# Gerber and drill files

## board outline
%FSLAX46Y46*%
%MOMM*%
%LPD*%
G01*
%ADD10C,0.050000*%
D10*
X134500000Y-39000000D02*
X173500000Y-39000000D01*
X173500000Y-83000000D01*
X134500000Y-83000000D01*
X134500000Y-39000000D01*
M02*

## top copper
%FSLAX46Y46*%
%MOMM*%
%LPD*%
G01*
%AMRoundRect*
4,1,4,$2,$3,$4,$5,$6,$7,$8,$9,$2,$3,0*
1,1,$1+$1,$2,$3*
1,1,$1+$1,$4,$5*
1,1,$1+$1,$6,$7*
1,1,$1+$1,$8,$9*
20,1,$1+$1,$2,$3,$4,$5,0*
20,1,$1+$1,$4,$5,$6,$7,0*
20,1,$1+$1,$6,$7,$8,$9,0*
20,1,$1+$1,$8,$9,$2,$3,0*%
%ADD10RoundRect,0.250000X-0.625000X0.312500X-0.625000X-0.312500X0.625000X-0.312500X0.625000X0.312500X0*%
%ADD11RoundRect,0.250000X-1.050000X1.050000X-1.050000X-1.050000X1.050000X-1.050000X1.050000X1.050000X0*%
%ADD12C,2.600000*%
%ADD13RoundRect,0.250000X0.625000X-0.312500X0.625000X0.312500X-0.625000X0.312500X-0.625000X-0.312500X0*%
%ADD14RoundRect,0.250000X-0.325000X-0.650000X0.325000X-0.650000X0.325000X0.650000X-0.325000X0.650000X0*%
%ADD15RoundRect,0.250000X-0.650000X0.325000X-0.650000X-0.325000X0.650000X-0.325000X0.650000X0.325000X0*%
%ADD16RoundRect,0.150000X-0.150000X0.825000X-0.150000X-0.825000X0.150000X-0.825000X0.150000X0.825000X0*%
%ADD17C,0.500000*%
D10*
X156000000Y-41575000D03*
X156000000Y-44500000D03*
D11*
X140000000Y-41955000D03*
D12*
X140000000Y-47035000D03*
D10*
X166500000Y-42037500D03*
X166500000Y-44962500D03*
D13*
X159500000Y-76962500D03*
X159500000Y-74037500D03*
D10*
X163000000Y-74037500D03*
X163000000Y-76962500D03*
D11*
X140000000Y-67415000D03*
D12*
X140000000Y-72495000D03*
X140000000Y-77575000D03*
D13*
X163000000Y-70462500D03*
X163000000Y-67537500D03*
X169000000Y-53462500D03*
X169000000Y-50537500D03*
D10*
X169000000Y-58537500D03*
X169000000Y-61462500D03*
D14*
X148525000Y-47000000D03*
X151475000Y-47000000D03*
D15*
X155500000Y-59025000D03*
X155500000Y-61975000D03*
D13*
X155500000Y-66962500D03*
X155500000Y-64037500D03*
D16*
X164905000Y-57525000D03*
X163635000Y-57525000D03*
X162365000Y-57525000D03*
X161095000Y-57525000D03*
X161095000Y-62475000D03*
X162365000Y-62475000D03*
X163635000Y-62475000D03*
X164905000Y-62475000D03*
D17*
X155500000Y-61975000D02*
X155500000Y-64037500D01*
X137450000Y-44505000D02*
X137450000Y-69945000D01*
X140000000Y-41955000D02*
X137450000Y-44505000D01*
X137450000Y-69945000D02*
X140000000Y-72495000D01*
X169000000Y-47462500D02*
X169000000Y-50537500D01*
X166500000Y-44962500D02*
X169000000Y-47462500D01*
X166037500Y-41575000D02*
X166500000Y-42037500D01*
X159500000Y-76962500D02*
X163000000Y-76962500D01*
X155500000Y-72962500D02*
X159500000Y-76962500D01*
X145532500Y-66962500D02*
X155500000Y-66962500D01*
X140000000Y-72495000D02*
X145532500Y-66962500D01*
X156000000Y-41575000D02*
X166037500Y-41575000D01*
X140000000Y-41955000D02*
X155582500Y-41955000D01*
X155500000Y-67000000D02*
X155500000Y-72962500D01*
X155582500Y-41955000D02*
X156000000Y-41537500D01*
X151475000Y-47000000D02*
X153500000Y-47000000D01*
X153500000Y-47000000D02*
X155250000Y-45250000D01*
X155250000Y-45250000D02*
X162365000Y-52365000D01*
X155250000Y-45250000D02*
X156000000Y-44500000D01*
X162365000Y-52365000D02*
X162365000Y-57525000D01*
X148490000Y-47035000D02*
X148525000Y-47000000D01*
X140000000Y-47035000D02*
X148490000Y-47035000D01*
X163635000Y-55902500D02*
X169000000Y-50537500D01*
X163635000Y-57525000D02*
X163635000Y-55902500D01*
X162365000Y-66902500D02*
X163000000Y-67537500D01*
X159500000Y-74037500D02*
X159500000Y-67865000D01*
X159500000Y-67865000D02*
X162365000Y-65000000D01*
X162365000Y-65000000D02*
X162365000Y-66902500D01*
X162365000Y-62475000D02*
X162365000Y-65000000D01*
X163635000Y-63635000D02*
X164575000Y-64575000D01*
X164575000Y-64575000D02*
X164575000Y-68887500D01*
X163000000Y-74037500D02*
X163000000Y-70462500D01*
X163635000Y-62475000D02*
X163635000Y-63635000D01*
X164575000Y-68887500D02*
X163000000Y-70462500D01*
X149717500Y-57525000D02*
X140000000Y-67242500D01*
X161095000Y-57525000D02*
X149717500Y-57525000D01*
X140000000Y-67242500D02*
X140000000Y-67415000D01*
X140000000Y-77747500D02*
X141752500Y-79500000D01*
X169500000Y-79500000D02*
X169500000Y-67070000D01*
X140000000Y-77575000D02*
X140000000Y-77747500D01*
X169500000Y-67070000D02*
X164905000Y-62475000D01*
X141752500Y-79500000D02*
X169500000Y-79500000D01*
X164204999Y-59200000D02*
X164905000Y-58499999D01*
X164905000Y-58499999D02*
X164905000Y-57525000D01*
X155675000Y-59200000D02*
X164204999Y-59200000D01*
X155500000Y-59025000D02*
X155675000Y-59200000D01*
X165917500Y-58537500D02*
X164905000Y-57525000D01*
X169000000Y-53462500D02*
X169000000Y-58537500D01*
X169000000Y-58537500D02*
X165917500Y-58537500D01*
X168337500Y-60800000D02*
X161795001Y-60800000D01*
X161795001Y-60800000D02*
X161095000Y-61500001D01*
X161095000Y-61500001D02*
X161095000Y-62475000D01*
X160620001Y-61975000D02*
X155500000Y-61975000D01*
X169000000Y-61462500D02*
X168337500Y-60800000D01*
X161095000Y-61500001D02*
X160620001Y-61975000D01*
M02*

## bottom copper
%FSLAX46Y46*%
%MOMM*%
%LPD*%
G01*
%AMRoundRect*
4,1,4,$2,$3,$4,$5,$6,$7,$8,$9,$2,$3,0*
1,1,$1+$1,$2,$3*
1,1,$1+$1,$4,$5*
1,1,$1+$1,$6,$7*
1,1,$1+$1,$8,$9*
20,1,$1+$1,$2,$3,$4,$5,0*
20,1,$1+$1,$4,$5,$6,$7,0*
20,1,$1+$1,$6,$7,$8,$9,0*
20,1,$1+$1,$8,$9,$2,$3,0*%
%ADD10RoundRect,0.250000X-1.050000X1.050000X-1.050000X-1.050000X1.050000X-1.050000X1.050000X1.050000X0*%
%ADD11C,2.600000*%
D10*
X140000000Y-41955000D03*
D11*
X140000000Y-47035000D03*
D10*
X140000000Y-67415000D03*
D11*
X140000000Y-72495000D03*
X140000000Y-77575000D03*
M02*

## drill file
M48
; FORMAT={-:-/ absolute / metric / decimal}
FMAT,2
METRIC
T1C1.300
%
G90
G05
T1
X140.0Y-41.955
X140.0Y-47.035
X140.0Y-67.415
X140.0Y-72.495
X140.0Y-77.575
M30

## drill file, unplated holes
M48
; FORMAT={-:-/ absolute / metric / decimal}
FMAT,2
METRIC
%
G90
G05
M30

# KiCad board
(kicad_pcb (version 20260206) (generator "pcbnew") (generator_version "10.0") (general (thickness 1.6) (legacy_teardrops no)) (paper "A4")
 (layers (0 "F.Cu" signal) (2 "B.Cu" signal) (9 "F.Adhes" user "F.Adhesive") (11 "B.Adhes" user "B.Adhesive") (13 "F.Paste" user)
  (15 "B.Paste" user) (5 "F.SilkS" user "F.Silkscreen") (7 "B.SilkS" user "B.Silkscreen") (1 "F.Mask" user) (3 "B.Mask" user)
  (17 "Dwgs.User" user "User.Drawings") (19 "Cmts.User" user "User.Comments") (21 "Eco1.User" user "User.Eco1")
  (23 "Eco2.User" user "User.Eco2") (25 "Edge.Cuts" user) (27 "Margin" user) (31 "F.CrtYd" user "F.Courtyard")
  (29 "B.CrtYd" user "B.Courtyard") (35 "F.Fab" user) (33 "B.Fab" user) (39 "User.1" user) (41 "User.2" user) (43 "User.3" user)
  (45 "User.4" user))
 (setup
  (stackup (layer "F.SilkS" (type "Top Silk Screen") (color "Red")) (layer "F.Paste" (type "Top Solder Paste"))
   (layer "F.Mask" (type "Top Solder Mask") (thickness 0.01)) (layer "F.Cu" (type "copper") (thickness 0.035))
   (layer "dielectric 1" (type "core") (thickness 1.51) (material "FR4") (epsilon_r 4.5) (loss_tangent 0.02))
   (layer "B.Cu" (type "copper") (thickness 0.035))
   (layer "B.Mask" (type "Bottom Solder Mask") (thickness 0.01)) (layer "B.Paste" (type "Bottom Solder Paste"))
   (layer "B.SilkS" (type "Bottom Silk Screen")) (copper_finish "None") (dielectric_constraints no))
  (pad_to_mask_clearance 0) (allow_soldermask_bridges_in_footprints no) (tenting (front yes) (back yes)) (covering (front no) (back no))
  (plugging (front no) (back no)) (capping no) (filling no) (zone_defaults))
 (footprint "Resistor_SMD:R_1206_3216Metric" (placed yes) (layer "F.Cu") (at 156 43.0375 -90)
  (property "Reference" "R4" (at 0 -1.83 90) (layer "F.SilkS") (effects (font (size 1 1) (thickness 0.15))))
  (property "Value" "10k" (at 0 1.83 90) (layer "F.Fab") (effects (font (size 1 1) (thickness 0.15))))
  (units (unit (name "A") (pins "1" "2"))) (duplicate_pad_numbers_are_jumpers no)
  (pad "1" smd roundrect (at -1.4625 0 270) (size 1.125 1.75) (layers "F.Cu" "F.Mask" "F.Paste") (roundrect_rratio 0.222222) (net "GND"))
  (pad "2" smd roundrect (at 1.4625 0 270) (size 1.125 1.75) (layers "F.Cu" "F.Mask" "F.Paste") (roundrect_rratio 0.222222)
   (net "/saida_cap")))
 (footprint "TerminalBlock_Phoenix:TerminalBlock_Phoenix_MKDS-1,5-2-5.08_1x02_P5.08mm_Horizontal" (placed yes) (layer "F.Cu")
  (at 140 41.955 -90)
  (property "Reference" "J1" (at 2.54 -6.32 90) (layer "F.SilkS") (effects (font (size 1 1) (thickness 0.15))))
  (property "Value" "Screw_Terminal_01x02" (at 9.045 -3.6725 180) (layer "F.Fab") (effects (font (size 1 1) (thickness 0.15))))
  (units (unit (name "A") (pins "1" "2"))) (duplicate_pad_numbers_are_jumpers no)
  (pad "1" thru_hole roundrect (at 0 0 270) (size 2.6 2.6) (drill 1.3) (layers "*.Cu" "*.Mask") (remove_unused_layers no)
   (roundrect_rratio 0.096154) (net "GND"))
  (pad "2" thru_hole circle (at 5.08 0 270) (size 2.6 2.6) (drill 1.3) (layers "*.Cu" "*.Mask") (remove_unused_layers no) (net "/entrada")))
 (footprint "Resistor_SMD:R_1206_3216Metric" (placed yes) (layer "F.Cu") (at 166.5 43.5 -90)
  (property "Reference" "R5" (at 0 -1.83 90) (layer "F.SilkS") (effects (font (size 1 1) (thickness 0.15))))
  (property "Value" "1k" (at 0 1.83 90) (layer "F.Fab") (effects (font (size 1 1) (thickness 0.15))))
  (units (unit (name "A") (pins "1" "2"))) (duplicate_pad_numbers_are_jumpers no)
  (pad "1" smd roundrect (at -1.4625 0 270) (size 1.125 1.75) (layers "F.Cu" "F.Mask" "F.Paste") (roundrect_rratio 0.222222) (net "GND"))
  (pad "2" smd roundrect (at 1.4625 0 270) (size 1.125 1.75) (layers "F.Cu" "F.Mask" "F.Paste") (roundrect_rratio 0.222222)
   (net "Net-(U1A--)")))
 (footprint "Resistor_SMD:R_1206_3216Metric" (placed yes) (layer "F.Cu") (at 159.5 75.5 90)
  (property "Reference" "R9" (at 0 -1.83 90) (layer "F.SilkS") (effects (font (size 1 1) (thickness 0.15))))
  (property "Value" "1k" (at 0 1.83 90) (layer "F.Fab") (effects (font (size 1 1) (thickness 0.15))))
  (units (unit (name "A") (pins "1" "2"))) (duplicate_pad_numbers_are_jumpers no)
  (pad "1" smd roundrect (at -1.4625 0 90) (size 1.125 1.75) (layers "F.Cu" "F.Mask" "F.Paste") (roundrect_rratio 0.222222) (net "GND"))
  (pad "2" smd roundrect (at 1.4625 0 90) (size 1.125 1.75) (layers "F.Cu" "F.Mask" "F.Paste") (roundrect_rratio 0.222222)
   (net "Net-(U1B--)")))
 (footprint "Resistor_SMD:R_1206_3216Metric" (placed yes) (layer "F.Cu") (at 163 75.5 -90)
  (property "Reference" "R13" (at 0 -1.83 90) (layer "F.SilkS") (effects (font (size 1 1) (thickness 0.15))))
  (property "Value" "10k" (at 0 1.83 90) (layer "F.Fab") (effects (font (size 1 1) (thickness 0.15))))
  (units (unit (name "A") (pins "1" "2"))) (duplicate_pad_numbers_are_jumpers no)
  (pad "1" smd roundrect (at -1.4625 0 270) (size 1.125 1.75) (layers "F.Cu" "F.Mask" "F.Paste") (roundrect_rratio 0.222222) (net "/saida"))
  (pad "2" smd roundrect (at 1.4625 0 270) (size 1.125 1.75) (layers "F.Cu" "F.Mask" "F.Paste") (roundrect_rratio 0.222222) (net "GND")))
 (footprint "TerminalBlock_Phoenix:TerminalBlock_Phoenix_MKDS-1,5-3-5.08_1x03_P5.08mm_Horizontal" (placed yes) (layer "F.Cu")
  (at 140 67.415 -90)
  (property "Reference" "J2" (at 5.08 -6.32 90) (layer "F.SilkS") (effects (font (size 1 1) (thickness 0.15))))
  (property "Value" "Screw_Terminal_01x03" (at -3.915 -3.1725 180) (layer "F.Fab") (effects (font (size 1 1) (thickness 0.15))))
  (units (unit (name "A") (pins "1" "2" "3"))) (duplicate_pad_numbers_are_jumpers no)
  (pad "1" thru_hole roundrect (at 0 0 270) (size 2.6 2.6) (drill 1.3) (layers "*.Cu" "*.Mask") (remove_unused_layers no)
   (roundrect_rratio 0.096154) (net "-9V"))
  (pad "2" thru_hole circle (at 5.08 0 270) (size 2.6 2.6) (drill 1.3) (layers "*.Cu" "*.Mask") (remove_unused_layers no) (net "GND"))
  (pad "3" thru_hole circle (at 10.16 0 270) (size 2.6 2.6) (drill 1.3) (layers "*.Cu" "*.Mask") (remove_unused_layers no) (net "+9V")))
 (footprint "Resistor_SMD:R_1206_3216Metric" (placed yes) (layer "F.Cu") (at 163 69 90)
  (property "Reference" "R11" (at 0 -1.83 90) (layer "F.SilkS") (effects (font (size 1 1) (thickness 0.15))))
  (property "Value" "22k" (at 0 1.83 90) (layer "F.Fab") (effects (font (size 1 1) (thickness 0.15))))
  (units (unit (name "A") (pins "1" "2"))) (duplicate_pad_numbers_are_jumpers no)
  (pad "1" smd roundrect (at -1.4625 0 90) (size 1.125 1.75) (layers "F.Cu" "F.Mask" "F.Paste") (roundrect_rratio 0.222222) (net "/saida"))
  (pad "2" smd roundrect (at 1.4625 0 90) (size 1.125 1.75) (layers "F.Cu" "F.Mask" "F.Paste") (roundrect_rratio 0.222222)
   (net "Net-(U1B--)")))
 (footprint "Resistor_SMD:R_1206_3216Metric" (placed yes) (layer "F.Cu") (at 169 52 90)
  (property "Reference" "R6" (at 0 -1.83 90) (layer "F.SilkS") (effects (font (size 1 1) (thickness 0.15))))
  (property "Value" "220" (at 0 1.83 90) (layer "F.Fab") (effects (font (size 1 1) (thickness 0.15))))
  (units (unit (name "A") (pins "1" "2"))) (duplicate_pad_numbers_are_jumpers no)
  (pad "1" smd roundrect (at -1.4625 0 90) (size 1.125 1.75) (layers "F.Cu" "F.Mask" "F.Paste") (roundrect_rratio 0.222222)
   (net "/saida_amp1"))
  (pad "2" smd roundrect (at 1.4625 0 90) (size 1.125 1.75) (layers "F.Cu" "F.Mask" "F.Paste") (roundrect_rratio 0.222222)
   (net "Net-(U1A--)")))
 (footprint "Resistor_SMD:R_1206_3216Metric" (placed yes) (layer "F.Cu") (at 169 60 -90)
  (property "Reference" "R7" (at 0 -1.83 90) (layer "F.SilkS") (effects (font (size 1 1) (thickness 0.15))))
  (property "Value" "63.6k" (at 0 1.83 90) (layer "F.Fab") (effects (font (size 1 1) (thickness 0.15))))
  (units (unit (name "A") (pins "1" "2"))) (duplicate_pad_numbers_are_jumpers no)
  (pad "1" smd roundrect (at -1.4625 0 270) (size 1.125 1.75) (layers "F.Cu" "F.Mask" "F.Paste") (roundrect_rratio 0.222222)
   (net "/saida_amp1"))
  (pad "2" smd roundrect (at 1.4625 0 270) (size 1.125 1.75) (layers "F.Cu" "F.Mask" "F.Paste") (roundrect_rratio 0.222222)
   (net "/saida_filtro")))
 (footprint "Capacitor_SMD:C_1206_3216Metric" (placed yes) (layer "F.Cu") (at 150 47)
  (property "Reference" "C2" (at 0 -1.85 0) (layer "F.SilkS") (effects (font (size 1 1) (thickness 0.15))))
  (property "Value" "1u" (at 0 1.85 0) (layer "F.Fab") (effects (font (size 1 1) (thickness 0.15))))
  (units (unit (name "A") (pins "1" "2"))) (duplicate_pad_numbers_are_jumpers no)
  (pad "1" smd roundrect (at -1.475 0) (size 1.15 1.8) (layers "F.Cu" "F.Mask" "F.Paste") (roundrect_rratio 0.217391) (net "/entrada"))
  (pad "2" smd roundrect (at 1.475 0) (size 1.15 1.8) (layers "F.Cu" "F.Mask" "F.Paste") (roundrect_rratio 0.217391) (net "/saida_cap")))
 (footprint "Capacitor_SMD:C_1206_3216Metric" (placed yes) (layer "F.Cu") (at 155.5 60.5 -90)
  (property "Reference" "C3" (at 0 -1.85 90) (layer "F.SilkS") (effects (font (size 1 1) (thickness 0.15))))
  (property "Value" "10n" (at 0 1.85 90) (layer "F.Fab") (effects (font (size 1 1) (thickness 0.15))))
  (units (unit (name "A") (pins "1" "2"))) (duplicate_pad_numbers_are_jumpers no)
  (pad "1" smd roundrect (at -1.475 0 270) (size 1.15 1.8) (layers "F.Cu" "F.Mask" "F.Paste") (roundrect_rratio 0.217391)
   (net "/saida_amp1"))
  (pad "2" smd roundrect (at 1.475 0 270) (size 1.15 1.8) (layers "F.Cu" "F.Mask" "F.Paste") (roundrect_rratio 0.217391)
   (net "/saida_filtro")))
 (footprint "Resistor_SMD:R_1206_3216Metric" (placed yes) (layer "F.Cu") (at 155.5 65.5 90)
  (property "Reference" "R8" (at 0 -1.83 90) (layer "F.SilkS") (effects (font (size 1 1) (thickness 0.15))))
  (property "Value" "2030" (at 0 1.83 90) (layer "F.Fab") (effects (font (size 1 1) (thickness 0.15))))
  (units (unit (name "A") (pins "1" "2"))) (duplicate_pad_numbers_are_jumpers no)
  (pad "1" smd roundrect (at -1.4625 0 90) (size 1.125 1.75) (layers "F.Cu" "F.Mask" "F.Paste") (roundrect_rratio 0.222222) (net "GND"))
  (pad "2" smd roundrect (at 1.4625 0 90) (size 1.125 1.75) (layers "F.Cu" "F.Mask" "F.Paste") (roundrect_rratio 0.222222)
   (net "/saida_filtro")))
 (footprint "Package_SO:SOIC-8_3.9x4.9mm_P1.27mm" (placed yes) (layer "F.Cu") (at 163 60 -90)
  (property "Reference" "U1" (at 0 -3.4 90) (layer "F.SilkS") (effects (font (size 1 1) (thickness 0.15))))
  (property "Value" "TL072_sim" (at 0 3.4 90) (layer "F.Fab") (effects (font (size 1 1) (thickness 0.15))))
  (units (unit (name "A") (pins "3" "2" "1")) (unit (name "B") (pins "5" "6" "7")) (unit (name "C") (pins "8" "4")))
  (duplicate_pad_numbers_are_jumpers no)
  (pad "1" smd roundrect (at -2.475 -1.905 270) (size 1.95 0.6) (layers "F.Cu" "F.Mask" "F.Paste") (roundrect_rratio 0.25)
   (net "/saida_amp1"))
  (pad "2" smd roundrect (at -2.475 -0.635 270) (size 1.95 0.6) (layers "F.Cu" "F.Mask" "F.Paste") (roundrect_rratio 0.25)
   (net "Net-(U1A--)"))
  (pad "3" smd roundrect (at -2.475 0.635 270) (size 1.95 0.6) (layers "F.Cu" "F.Mask" "F.Paste") (roundrect_rratio 0.25) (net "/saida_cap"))
  (pad "4" smd roundrect (at -2.475 1.905 270) (size 1.95 0.6) (layers "F.Cu" "F.Mask" "F.Paste") (roundrect_rratio 0.25) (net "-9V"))
  (pad "5" smd roundrect (at 2.475 1.905 270) (size 1.95 0.6) (layers "F.Cu" "F.Mask" "F.Paste") (roundrect_rratio 0.25)
   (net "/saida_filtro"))
  (pad "6" smd roundrect (at 2.475 0.635 270) (size 1.95 0.6) (layers "F.Cu" "F.Mask" "F.Paste") (roundrect_rratio 0.25) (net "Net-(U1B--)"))
  (pad "7" smd roundrect (at 2.475 -0.635 270) (size 1.95 0.6) (layers "F.Cu" "F.Mask" "F.Paste") (roundrect_rratio 0.25) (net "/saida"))
  (pad "8" smd roundrect (at 2.475 -1.905 270) (size 1.95 0.6) (layers "F.Cu" "F.Mask" "F.Paste") (roundrect_rratio 0.25) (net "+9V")))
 (gr_rect (start 134.5 39) (end 173.5 83) (stroke (width 0.05) (type default)) (fill no) (layer "Edge.Cuts"))
 (segment (start 137.45 69.945) (end 140 72.495) (width 0.5) (layer "F.Cu") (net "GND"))
 (segment (start 140 41.955) (end 137.45 44.505) (width 0.5) (layer "F.Cu") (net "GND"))
 (segment (start 166.0375 41.575) (end 166.5 42.0375) (width 0.5) (layer "F.Cu") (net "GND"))
 (segment (start 159.5 76.9625) (end 163 76.9625) (width 0.5) (layer "F.Cu") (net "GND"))
 (segment (start 137.45 44.505) (end 137.45 69.945) (width 0.5) (layer "F.Cu") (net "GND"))
 (segment (start 155.5 72.9625) (end 159.5 76.9625) (width 0.5) (layer "F.Cu") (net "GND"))
 (segment (start 145.5325 66.9625) (end 155.5 66.9625) (width 0.5) (layer "F.Cu") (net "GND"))
 (segment (start 140 72.495) (end 145.5325 66.9625) (width 0.5) (layer "F.Cu") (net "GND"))
 (segment (start 156 41.575) (end 166.0375 41.575) (width 0.5) (layer "F.Cu") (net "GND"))
 (segment (start 140 41.955) (end 155.5825 41.955) (width 0.5) (layer "F.Cu") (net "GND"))
 (segment (start 155.5 67) (end 155.5 72.9625) (width 0.5) (layer "F.Cu") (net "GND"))
 (segment (start 155.5825 41.955) (end 156 41.5375) (width 0.5) (layer "F.Cu") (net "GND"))
 (segment (start 151.475 47) (end 153.5 47) (width 0.5) (layer "F.Cu") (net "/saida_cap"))
 (segment (start 153.5 47) (end 155.25 45.25) (width 0.5) (layer "F.Cu") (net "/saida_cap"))
 (segment (start 155.25 45.25) (end 162.365 52.365) (width 0.5) (layer "F.Cu") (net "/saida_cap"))
 (segment (start 155.25 45.25) (end 156 44.5) (width 0.5) (layer "F.Cu") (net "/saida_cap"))
 (segment (start 162.365 52.365) (end 162.365 57.525) (width 0.5) (layer "F.Cu") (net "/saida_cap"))
 (segment (start 148.49 47.035) (end 148.525 47) (width 0.5) (layer "F.Cu") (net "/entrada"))
 (segment (start 140 47.035) (end 148.49 47.035) (width 0.5) (layer "F.Cu") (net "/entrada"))
 (segment (start 163.635 55.9025) (end 169 50.5375) (width 0.5) (layer "F.Cu") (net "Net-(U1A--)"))
 (segment (start 169 47.4625) (end 169 50.5375) (width 0.5) (layer "F.Cu") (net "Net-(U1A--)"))
 (segment (start 163.635 57.525) (end 163.635 55.9025) (width 0.5) (layer "F.Cu") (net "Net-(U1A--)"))
 (segment (start 166.5 44.9625) (end 169 47.4625) (width 0.5) (layer "F.Cu") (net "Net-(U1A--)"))
 (segment (start 162.365 66.9025) (end 163 67.5375) (width 0.5) (layer "F.Cu") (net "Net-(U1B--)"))
 (segment (start 159.5 74.0375) (end 159.5 67.865) (width 0.5) (layer "F.Cu") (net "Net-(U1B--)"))
 (segment (start 159.5 67.865) (end 162.365 65) (width 0.5) (layer "F.Cu") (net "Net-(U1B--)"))
 (segment (start 162.365 65) (end 162.365 66.9025) (width 0.5) (layer "F.Cu") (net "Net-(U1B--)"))
 (segment (start 162.365 62.475) (end 162.365 65) (width 0.5) (layer "F.Cu") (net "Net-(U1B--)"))
 (segment (start 163.635 63.635) (end 164.575 64.575) (width 0.5) (layer "F.Cu") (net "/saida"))
 (segment (start 164.575 64.575) (end 164.575 68.8875) (width 0.5) (layer "F.Cu") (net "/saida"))
 (segment (start 163 74.0375) (end 163 70.4625) (width 0.5) (layer "F.Cu") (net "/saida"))
 (segment (start 163.635 62.475) (end 163.635 63.635) (width 0.5) (layer "F.Cu") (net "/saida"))
 (segment (start 164.575 68.8875) (end 163 70.4625) (width 0.5) (layer "F.Cu") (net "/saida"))
 (segment (start 149.7175 57.525) (end 140 67.2425) (width 0.5) (layer "F.Cu") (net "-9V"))
 (segment (start 161.095 57.525) (end 149.7175 57.525) (width 0.5) (layer "F.Cu") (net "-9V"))
 (segment (start 140 67.2425) (end 140 67.415) (width 0.5) (layer "F.Cu") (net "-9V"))
 (segment (start 140 77.7475) (end 141.7525 79.5) (width 0.5) (layer "F.Cu") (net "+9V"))
 (segment (start 169.5 79.5) (end 169.5 67.07) (width 0.5) (layer "F.Cu") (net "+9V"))
 (segment (start 140 77.575) (end 140 77.7475) (width 0.5) (layer "F.Cu") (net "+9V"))
 (segment (start 169.5 67.07) (end 164.905 62.475) (width 0.5) (layer "F.Cu") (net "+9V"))
 (segment (start 141.7525 79.5) (end 169.5 79.5) (width 0.5) (layer "F.Cu") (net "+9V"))
 (segment (start 164.204999 59.2) (end 164.905 58.499999) (width 0.5) (layer "F.Cu") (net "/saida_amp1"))
 (segment (start 164.905 58.499999) (end 164.905 57.525) (width 0.5) (layer "F.Cu") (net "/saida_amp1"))
 (segment (start 155.675 59.2) (end 164.204999 59.2) (width 0.5) (layer "F.Cu") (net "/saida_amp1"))
 (segment (start 155.5 59.025) (end 155.675 59.2) (width 0.5) (layer "F.Cu") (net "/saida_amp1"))
 (segment (start 165.9175 58.5375) (end 164.905 57.525) (width 0.5) (layer "F.Cu") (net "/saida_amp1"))
 (segment (start 169 53.4625) (end 169 58.5375) (width 0.5) (layer "F.Cu") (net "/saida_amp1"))
 (segment (start 169 58.5375) (end 165.9175 58.5375) (width 0.5) (layer "F.Cu") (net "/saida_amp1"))
 (segment (start 168.3375 60.8) (end 161.795001 60.8) (width 0.5) (layer "F.Cu") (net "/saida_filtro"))
 (segment (start 161.795001 60.8) (end 161.095 61.500001) (width 0.5) (layer "F.Cu") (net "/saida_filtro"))
 (segment (start 161.095 61.500001) (end 161.095 62.475) (width 0.5) (layer "F.Cu") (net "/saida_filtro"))
 (segment (start 155.5 61.975) (end 155.5 64.0375) (width 0.5) (layer "F.Cu") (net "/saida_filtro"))
 (segment (start 160.620001 61.975) (end 155.5 61.975) (width 0.5) (layer "F.Cu") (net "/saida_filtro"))
 (segment (start 169 61.4625) (end 168.3375 60.8) (width 0.5) (layer "F.Cu") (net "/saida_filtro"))
 (segment (start 161.095 61.500001) (end 160.620001 61.975) (width 0.5) (layer "F.Cu") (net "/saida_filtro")))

